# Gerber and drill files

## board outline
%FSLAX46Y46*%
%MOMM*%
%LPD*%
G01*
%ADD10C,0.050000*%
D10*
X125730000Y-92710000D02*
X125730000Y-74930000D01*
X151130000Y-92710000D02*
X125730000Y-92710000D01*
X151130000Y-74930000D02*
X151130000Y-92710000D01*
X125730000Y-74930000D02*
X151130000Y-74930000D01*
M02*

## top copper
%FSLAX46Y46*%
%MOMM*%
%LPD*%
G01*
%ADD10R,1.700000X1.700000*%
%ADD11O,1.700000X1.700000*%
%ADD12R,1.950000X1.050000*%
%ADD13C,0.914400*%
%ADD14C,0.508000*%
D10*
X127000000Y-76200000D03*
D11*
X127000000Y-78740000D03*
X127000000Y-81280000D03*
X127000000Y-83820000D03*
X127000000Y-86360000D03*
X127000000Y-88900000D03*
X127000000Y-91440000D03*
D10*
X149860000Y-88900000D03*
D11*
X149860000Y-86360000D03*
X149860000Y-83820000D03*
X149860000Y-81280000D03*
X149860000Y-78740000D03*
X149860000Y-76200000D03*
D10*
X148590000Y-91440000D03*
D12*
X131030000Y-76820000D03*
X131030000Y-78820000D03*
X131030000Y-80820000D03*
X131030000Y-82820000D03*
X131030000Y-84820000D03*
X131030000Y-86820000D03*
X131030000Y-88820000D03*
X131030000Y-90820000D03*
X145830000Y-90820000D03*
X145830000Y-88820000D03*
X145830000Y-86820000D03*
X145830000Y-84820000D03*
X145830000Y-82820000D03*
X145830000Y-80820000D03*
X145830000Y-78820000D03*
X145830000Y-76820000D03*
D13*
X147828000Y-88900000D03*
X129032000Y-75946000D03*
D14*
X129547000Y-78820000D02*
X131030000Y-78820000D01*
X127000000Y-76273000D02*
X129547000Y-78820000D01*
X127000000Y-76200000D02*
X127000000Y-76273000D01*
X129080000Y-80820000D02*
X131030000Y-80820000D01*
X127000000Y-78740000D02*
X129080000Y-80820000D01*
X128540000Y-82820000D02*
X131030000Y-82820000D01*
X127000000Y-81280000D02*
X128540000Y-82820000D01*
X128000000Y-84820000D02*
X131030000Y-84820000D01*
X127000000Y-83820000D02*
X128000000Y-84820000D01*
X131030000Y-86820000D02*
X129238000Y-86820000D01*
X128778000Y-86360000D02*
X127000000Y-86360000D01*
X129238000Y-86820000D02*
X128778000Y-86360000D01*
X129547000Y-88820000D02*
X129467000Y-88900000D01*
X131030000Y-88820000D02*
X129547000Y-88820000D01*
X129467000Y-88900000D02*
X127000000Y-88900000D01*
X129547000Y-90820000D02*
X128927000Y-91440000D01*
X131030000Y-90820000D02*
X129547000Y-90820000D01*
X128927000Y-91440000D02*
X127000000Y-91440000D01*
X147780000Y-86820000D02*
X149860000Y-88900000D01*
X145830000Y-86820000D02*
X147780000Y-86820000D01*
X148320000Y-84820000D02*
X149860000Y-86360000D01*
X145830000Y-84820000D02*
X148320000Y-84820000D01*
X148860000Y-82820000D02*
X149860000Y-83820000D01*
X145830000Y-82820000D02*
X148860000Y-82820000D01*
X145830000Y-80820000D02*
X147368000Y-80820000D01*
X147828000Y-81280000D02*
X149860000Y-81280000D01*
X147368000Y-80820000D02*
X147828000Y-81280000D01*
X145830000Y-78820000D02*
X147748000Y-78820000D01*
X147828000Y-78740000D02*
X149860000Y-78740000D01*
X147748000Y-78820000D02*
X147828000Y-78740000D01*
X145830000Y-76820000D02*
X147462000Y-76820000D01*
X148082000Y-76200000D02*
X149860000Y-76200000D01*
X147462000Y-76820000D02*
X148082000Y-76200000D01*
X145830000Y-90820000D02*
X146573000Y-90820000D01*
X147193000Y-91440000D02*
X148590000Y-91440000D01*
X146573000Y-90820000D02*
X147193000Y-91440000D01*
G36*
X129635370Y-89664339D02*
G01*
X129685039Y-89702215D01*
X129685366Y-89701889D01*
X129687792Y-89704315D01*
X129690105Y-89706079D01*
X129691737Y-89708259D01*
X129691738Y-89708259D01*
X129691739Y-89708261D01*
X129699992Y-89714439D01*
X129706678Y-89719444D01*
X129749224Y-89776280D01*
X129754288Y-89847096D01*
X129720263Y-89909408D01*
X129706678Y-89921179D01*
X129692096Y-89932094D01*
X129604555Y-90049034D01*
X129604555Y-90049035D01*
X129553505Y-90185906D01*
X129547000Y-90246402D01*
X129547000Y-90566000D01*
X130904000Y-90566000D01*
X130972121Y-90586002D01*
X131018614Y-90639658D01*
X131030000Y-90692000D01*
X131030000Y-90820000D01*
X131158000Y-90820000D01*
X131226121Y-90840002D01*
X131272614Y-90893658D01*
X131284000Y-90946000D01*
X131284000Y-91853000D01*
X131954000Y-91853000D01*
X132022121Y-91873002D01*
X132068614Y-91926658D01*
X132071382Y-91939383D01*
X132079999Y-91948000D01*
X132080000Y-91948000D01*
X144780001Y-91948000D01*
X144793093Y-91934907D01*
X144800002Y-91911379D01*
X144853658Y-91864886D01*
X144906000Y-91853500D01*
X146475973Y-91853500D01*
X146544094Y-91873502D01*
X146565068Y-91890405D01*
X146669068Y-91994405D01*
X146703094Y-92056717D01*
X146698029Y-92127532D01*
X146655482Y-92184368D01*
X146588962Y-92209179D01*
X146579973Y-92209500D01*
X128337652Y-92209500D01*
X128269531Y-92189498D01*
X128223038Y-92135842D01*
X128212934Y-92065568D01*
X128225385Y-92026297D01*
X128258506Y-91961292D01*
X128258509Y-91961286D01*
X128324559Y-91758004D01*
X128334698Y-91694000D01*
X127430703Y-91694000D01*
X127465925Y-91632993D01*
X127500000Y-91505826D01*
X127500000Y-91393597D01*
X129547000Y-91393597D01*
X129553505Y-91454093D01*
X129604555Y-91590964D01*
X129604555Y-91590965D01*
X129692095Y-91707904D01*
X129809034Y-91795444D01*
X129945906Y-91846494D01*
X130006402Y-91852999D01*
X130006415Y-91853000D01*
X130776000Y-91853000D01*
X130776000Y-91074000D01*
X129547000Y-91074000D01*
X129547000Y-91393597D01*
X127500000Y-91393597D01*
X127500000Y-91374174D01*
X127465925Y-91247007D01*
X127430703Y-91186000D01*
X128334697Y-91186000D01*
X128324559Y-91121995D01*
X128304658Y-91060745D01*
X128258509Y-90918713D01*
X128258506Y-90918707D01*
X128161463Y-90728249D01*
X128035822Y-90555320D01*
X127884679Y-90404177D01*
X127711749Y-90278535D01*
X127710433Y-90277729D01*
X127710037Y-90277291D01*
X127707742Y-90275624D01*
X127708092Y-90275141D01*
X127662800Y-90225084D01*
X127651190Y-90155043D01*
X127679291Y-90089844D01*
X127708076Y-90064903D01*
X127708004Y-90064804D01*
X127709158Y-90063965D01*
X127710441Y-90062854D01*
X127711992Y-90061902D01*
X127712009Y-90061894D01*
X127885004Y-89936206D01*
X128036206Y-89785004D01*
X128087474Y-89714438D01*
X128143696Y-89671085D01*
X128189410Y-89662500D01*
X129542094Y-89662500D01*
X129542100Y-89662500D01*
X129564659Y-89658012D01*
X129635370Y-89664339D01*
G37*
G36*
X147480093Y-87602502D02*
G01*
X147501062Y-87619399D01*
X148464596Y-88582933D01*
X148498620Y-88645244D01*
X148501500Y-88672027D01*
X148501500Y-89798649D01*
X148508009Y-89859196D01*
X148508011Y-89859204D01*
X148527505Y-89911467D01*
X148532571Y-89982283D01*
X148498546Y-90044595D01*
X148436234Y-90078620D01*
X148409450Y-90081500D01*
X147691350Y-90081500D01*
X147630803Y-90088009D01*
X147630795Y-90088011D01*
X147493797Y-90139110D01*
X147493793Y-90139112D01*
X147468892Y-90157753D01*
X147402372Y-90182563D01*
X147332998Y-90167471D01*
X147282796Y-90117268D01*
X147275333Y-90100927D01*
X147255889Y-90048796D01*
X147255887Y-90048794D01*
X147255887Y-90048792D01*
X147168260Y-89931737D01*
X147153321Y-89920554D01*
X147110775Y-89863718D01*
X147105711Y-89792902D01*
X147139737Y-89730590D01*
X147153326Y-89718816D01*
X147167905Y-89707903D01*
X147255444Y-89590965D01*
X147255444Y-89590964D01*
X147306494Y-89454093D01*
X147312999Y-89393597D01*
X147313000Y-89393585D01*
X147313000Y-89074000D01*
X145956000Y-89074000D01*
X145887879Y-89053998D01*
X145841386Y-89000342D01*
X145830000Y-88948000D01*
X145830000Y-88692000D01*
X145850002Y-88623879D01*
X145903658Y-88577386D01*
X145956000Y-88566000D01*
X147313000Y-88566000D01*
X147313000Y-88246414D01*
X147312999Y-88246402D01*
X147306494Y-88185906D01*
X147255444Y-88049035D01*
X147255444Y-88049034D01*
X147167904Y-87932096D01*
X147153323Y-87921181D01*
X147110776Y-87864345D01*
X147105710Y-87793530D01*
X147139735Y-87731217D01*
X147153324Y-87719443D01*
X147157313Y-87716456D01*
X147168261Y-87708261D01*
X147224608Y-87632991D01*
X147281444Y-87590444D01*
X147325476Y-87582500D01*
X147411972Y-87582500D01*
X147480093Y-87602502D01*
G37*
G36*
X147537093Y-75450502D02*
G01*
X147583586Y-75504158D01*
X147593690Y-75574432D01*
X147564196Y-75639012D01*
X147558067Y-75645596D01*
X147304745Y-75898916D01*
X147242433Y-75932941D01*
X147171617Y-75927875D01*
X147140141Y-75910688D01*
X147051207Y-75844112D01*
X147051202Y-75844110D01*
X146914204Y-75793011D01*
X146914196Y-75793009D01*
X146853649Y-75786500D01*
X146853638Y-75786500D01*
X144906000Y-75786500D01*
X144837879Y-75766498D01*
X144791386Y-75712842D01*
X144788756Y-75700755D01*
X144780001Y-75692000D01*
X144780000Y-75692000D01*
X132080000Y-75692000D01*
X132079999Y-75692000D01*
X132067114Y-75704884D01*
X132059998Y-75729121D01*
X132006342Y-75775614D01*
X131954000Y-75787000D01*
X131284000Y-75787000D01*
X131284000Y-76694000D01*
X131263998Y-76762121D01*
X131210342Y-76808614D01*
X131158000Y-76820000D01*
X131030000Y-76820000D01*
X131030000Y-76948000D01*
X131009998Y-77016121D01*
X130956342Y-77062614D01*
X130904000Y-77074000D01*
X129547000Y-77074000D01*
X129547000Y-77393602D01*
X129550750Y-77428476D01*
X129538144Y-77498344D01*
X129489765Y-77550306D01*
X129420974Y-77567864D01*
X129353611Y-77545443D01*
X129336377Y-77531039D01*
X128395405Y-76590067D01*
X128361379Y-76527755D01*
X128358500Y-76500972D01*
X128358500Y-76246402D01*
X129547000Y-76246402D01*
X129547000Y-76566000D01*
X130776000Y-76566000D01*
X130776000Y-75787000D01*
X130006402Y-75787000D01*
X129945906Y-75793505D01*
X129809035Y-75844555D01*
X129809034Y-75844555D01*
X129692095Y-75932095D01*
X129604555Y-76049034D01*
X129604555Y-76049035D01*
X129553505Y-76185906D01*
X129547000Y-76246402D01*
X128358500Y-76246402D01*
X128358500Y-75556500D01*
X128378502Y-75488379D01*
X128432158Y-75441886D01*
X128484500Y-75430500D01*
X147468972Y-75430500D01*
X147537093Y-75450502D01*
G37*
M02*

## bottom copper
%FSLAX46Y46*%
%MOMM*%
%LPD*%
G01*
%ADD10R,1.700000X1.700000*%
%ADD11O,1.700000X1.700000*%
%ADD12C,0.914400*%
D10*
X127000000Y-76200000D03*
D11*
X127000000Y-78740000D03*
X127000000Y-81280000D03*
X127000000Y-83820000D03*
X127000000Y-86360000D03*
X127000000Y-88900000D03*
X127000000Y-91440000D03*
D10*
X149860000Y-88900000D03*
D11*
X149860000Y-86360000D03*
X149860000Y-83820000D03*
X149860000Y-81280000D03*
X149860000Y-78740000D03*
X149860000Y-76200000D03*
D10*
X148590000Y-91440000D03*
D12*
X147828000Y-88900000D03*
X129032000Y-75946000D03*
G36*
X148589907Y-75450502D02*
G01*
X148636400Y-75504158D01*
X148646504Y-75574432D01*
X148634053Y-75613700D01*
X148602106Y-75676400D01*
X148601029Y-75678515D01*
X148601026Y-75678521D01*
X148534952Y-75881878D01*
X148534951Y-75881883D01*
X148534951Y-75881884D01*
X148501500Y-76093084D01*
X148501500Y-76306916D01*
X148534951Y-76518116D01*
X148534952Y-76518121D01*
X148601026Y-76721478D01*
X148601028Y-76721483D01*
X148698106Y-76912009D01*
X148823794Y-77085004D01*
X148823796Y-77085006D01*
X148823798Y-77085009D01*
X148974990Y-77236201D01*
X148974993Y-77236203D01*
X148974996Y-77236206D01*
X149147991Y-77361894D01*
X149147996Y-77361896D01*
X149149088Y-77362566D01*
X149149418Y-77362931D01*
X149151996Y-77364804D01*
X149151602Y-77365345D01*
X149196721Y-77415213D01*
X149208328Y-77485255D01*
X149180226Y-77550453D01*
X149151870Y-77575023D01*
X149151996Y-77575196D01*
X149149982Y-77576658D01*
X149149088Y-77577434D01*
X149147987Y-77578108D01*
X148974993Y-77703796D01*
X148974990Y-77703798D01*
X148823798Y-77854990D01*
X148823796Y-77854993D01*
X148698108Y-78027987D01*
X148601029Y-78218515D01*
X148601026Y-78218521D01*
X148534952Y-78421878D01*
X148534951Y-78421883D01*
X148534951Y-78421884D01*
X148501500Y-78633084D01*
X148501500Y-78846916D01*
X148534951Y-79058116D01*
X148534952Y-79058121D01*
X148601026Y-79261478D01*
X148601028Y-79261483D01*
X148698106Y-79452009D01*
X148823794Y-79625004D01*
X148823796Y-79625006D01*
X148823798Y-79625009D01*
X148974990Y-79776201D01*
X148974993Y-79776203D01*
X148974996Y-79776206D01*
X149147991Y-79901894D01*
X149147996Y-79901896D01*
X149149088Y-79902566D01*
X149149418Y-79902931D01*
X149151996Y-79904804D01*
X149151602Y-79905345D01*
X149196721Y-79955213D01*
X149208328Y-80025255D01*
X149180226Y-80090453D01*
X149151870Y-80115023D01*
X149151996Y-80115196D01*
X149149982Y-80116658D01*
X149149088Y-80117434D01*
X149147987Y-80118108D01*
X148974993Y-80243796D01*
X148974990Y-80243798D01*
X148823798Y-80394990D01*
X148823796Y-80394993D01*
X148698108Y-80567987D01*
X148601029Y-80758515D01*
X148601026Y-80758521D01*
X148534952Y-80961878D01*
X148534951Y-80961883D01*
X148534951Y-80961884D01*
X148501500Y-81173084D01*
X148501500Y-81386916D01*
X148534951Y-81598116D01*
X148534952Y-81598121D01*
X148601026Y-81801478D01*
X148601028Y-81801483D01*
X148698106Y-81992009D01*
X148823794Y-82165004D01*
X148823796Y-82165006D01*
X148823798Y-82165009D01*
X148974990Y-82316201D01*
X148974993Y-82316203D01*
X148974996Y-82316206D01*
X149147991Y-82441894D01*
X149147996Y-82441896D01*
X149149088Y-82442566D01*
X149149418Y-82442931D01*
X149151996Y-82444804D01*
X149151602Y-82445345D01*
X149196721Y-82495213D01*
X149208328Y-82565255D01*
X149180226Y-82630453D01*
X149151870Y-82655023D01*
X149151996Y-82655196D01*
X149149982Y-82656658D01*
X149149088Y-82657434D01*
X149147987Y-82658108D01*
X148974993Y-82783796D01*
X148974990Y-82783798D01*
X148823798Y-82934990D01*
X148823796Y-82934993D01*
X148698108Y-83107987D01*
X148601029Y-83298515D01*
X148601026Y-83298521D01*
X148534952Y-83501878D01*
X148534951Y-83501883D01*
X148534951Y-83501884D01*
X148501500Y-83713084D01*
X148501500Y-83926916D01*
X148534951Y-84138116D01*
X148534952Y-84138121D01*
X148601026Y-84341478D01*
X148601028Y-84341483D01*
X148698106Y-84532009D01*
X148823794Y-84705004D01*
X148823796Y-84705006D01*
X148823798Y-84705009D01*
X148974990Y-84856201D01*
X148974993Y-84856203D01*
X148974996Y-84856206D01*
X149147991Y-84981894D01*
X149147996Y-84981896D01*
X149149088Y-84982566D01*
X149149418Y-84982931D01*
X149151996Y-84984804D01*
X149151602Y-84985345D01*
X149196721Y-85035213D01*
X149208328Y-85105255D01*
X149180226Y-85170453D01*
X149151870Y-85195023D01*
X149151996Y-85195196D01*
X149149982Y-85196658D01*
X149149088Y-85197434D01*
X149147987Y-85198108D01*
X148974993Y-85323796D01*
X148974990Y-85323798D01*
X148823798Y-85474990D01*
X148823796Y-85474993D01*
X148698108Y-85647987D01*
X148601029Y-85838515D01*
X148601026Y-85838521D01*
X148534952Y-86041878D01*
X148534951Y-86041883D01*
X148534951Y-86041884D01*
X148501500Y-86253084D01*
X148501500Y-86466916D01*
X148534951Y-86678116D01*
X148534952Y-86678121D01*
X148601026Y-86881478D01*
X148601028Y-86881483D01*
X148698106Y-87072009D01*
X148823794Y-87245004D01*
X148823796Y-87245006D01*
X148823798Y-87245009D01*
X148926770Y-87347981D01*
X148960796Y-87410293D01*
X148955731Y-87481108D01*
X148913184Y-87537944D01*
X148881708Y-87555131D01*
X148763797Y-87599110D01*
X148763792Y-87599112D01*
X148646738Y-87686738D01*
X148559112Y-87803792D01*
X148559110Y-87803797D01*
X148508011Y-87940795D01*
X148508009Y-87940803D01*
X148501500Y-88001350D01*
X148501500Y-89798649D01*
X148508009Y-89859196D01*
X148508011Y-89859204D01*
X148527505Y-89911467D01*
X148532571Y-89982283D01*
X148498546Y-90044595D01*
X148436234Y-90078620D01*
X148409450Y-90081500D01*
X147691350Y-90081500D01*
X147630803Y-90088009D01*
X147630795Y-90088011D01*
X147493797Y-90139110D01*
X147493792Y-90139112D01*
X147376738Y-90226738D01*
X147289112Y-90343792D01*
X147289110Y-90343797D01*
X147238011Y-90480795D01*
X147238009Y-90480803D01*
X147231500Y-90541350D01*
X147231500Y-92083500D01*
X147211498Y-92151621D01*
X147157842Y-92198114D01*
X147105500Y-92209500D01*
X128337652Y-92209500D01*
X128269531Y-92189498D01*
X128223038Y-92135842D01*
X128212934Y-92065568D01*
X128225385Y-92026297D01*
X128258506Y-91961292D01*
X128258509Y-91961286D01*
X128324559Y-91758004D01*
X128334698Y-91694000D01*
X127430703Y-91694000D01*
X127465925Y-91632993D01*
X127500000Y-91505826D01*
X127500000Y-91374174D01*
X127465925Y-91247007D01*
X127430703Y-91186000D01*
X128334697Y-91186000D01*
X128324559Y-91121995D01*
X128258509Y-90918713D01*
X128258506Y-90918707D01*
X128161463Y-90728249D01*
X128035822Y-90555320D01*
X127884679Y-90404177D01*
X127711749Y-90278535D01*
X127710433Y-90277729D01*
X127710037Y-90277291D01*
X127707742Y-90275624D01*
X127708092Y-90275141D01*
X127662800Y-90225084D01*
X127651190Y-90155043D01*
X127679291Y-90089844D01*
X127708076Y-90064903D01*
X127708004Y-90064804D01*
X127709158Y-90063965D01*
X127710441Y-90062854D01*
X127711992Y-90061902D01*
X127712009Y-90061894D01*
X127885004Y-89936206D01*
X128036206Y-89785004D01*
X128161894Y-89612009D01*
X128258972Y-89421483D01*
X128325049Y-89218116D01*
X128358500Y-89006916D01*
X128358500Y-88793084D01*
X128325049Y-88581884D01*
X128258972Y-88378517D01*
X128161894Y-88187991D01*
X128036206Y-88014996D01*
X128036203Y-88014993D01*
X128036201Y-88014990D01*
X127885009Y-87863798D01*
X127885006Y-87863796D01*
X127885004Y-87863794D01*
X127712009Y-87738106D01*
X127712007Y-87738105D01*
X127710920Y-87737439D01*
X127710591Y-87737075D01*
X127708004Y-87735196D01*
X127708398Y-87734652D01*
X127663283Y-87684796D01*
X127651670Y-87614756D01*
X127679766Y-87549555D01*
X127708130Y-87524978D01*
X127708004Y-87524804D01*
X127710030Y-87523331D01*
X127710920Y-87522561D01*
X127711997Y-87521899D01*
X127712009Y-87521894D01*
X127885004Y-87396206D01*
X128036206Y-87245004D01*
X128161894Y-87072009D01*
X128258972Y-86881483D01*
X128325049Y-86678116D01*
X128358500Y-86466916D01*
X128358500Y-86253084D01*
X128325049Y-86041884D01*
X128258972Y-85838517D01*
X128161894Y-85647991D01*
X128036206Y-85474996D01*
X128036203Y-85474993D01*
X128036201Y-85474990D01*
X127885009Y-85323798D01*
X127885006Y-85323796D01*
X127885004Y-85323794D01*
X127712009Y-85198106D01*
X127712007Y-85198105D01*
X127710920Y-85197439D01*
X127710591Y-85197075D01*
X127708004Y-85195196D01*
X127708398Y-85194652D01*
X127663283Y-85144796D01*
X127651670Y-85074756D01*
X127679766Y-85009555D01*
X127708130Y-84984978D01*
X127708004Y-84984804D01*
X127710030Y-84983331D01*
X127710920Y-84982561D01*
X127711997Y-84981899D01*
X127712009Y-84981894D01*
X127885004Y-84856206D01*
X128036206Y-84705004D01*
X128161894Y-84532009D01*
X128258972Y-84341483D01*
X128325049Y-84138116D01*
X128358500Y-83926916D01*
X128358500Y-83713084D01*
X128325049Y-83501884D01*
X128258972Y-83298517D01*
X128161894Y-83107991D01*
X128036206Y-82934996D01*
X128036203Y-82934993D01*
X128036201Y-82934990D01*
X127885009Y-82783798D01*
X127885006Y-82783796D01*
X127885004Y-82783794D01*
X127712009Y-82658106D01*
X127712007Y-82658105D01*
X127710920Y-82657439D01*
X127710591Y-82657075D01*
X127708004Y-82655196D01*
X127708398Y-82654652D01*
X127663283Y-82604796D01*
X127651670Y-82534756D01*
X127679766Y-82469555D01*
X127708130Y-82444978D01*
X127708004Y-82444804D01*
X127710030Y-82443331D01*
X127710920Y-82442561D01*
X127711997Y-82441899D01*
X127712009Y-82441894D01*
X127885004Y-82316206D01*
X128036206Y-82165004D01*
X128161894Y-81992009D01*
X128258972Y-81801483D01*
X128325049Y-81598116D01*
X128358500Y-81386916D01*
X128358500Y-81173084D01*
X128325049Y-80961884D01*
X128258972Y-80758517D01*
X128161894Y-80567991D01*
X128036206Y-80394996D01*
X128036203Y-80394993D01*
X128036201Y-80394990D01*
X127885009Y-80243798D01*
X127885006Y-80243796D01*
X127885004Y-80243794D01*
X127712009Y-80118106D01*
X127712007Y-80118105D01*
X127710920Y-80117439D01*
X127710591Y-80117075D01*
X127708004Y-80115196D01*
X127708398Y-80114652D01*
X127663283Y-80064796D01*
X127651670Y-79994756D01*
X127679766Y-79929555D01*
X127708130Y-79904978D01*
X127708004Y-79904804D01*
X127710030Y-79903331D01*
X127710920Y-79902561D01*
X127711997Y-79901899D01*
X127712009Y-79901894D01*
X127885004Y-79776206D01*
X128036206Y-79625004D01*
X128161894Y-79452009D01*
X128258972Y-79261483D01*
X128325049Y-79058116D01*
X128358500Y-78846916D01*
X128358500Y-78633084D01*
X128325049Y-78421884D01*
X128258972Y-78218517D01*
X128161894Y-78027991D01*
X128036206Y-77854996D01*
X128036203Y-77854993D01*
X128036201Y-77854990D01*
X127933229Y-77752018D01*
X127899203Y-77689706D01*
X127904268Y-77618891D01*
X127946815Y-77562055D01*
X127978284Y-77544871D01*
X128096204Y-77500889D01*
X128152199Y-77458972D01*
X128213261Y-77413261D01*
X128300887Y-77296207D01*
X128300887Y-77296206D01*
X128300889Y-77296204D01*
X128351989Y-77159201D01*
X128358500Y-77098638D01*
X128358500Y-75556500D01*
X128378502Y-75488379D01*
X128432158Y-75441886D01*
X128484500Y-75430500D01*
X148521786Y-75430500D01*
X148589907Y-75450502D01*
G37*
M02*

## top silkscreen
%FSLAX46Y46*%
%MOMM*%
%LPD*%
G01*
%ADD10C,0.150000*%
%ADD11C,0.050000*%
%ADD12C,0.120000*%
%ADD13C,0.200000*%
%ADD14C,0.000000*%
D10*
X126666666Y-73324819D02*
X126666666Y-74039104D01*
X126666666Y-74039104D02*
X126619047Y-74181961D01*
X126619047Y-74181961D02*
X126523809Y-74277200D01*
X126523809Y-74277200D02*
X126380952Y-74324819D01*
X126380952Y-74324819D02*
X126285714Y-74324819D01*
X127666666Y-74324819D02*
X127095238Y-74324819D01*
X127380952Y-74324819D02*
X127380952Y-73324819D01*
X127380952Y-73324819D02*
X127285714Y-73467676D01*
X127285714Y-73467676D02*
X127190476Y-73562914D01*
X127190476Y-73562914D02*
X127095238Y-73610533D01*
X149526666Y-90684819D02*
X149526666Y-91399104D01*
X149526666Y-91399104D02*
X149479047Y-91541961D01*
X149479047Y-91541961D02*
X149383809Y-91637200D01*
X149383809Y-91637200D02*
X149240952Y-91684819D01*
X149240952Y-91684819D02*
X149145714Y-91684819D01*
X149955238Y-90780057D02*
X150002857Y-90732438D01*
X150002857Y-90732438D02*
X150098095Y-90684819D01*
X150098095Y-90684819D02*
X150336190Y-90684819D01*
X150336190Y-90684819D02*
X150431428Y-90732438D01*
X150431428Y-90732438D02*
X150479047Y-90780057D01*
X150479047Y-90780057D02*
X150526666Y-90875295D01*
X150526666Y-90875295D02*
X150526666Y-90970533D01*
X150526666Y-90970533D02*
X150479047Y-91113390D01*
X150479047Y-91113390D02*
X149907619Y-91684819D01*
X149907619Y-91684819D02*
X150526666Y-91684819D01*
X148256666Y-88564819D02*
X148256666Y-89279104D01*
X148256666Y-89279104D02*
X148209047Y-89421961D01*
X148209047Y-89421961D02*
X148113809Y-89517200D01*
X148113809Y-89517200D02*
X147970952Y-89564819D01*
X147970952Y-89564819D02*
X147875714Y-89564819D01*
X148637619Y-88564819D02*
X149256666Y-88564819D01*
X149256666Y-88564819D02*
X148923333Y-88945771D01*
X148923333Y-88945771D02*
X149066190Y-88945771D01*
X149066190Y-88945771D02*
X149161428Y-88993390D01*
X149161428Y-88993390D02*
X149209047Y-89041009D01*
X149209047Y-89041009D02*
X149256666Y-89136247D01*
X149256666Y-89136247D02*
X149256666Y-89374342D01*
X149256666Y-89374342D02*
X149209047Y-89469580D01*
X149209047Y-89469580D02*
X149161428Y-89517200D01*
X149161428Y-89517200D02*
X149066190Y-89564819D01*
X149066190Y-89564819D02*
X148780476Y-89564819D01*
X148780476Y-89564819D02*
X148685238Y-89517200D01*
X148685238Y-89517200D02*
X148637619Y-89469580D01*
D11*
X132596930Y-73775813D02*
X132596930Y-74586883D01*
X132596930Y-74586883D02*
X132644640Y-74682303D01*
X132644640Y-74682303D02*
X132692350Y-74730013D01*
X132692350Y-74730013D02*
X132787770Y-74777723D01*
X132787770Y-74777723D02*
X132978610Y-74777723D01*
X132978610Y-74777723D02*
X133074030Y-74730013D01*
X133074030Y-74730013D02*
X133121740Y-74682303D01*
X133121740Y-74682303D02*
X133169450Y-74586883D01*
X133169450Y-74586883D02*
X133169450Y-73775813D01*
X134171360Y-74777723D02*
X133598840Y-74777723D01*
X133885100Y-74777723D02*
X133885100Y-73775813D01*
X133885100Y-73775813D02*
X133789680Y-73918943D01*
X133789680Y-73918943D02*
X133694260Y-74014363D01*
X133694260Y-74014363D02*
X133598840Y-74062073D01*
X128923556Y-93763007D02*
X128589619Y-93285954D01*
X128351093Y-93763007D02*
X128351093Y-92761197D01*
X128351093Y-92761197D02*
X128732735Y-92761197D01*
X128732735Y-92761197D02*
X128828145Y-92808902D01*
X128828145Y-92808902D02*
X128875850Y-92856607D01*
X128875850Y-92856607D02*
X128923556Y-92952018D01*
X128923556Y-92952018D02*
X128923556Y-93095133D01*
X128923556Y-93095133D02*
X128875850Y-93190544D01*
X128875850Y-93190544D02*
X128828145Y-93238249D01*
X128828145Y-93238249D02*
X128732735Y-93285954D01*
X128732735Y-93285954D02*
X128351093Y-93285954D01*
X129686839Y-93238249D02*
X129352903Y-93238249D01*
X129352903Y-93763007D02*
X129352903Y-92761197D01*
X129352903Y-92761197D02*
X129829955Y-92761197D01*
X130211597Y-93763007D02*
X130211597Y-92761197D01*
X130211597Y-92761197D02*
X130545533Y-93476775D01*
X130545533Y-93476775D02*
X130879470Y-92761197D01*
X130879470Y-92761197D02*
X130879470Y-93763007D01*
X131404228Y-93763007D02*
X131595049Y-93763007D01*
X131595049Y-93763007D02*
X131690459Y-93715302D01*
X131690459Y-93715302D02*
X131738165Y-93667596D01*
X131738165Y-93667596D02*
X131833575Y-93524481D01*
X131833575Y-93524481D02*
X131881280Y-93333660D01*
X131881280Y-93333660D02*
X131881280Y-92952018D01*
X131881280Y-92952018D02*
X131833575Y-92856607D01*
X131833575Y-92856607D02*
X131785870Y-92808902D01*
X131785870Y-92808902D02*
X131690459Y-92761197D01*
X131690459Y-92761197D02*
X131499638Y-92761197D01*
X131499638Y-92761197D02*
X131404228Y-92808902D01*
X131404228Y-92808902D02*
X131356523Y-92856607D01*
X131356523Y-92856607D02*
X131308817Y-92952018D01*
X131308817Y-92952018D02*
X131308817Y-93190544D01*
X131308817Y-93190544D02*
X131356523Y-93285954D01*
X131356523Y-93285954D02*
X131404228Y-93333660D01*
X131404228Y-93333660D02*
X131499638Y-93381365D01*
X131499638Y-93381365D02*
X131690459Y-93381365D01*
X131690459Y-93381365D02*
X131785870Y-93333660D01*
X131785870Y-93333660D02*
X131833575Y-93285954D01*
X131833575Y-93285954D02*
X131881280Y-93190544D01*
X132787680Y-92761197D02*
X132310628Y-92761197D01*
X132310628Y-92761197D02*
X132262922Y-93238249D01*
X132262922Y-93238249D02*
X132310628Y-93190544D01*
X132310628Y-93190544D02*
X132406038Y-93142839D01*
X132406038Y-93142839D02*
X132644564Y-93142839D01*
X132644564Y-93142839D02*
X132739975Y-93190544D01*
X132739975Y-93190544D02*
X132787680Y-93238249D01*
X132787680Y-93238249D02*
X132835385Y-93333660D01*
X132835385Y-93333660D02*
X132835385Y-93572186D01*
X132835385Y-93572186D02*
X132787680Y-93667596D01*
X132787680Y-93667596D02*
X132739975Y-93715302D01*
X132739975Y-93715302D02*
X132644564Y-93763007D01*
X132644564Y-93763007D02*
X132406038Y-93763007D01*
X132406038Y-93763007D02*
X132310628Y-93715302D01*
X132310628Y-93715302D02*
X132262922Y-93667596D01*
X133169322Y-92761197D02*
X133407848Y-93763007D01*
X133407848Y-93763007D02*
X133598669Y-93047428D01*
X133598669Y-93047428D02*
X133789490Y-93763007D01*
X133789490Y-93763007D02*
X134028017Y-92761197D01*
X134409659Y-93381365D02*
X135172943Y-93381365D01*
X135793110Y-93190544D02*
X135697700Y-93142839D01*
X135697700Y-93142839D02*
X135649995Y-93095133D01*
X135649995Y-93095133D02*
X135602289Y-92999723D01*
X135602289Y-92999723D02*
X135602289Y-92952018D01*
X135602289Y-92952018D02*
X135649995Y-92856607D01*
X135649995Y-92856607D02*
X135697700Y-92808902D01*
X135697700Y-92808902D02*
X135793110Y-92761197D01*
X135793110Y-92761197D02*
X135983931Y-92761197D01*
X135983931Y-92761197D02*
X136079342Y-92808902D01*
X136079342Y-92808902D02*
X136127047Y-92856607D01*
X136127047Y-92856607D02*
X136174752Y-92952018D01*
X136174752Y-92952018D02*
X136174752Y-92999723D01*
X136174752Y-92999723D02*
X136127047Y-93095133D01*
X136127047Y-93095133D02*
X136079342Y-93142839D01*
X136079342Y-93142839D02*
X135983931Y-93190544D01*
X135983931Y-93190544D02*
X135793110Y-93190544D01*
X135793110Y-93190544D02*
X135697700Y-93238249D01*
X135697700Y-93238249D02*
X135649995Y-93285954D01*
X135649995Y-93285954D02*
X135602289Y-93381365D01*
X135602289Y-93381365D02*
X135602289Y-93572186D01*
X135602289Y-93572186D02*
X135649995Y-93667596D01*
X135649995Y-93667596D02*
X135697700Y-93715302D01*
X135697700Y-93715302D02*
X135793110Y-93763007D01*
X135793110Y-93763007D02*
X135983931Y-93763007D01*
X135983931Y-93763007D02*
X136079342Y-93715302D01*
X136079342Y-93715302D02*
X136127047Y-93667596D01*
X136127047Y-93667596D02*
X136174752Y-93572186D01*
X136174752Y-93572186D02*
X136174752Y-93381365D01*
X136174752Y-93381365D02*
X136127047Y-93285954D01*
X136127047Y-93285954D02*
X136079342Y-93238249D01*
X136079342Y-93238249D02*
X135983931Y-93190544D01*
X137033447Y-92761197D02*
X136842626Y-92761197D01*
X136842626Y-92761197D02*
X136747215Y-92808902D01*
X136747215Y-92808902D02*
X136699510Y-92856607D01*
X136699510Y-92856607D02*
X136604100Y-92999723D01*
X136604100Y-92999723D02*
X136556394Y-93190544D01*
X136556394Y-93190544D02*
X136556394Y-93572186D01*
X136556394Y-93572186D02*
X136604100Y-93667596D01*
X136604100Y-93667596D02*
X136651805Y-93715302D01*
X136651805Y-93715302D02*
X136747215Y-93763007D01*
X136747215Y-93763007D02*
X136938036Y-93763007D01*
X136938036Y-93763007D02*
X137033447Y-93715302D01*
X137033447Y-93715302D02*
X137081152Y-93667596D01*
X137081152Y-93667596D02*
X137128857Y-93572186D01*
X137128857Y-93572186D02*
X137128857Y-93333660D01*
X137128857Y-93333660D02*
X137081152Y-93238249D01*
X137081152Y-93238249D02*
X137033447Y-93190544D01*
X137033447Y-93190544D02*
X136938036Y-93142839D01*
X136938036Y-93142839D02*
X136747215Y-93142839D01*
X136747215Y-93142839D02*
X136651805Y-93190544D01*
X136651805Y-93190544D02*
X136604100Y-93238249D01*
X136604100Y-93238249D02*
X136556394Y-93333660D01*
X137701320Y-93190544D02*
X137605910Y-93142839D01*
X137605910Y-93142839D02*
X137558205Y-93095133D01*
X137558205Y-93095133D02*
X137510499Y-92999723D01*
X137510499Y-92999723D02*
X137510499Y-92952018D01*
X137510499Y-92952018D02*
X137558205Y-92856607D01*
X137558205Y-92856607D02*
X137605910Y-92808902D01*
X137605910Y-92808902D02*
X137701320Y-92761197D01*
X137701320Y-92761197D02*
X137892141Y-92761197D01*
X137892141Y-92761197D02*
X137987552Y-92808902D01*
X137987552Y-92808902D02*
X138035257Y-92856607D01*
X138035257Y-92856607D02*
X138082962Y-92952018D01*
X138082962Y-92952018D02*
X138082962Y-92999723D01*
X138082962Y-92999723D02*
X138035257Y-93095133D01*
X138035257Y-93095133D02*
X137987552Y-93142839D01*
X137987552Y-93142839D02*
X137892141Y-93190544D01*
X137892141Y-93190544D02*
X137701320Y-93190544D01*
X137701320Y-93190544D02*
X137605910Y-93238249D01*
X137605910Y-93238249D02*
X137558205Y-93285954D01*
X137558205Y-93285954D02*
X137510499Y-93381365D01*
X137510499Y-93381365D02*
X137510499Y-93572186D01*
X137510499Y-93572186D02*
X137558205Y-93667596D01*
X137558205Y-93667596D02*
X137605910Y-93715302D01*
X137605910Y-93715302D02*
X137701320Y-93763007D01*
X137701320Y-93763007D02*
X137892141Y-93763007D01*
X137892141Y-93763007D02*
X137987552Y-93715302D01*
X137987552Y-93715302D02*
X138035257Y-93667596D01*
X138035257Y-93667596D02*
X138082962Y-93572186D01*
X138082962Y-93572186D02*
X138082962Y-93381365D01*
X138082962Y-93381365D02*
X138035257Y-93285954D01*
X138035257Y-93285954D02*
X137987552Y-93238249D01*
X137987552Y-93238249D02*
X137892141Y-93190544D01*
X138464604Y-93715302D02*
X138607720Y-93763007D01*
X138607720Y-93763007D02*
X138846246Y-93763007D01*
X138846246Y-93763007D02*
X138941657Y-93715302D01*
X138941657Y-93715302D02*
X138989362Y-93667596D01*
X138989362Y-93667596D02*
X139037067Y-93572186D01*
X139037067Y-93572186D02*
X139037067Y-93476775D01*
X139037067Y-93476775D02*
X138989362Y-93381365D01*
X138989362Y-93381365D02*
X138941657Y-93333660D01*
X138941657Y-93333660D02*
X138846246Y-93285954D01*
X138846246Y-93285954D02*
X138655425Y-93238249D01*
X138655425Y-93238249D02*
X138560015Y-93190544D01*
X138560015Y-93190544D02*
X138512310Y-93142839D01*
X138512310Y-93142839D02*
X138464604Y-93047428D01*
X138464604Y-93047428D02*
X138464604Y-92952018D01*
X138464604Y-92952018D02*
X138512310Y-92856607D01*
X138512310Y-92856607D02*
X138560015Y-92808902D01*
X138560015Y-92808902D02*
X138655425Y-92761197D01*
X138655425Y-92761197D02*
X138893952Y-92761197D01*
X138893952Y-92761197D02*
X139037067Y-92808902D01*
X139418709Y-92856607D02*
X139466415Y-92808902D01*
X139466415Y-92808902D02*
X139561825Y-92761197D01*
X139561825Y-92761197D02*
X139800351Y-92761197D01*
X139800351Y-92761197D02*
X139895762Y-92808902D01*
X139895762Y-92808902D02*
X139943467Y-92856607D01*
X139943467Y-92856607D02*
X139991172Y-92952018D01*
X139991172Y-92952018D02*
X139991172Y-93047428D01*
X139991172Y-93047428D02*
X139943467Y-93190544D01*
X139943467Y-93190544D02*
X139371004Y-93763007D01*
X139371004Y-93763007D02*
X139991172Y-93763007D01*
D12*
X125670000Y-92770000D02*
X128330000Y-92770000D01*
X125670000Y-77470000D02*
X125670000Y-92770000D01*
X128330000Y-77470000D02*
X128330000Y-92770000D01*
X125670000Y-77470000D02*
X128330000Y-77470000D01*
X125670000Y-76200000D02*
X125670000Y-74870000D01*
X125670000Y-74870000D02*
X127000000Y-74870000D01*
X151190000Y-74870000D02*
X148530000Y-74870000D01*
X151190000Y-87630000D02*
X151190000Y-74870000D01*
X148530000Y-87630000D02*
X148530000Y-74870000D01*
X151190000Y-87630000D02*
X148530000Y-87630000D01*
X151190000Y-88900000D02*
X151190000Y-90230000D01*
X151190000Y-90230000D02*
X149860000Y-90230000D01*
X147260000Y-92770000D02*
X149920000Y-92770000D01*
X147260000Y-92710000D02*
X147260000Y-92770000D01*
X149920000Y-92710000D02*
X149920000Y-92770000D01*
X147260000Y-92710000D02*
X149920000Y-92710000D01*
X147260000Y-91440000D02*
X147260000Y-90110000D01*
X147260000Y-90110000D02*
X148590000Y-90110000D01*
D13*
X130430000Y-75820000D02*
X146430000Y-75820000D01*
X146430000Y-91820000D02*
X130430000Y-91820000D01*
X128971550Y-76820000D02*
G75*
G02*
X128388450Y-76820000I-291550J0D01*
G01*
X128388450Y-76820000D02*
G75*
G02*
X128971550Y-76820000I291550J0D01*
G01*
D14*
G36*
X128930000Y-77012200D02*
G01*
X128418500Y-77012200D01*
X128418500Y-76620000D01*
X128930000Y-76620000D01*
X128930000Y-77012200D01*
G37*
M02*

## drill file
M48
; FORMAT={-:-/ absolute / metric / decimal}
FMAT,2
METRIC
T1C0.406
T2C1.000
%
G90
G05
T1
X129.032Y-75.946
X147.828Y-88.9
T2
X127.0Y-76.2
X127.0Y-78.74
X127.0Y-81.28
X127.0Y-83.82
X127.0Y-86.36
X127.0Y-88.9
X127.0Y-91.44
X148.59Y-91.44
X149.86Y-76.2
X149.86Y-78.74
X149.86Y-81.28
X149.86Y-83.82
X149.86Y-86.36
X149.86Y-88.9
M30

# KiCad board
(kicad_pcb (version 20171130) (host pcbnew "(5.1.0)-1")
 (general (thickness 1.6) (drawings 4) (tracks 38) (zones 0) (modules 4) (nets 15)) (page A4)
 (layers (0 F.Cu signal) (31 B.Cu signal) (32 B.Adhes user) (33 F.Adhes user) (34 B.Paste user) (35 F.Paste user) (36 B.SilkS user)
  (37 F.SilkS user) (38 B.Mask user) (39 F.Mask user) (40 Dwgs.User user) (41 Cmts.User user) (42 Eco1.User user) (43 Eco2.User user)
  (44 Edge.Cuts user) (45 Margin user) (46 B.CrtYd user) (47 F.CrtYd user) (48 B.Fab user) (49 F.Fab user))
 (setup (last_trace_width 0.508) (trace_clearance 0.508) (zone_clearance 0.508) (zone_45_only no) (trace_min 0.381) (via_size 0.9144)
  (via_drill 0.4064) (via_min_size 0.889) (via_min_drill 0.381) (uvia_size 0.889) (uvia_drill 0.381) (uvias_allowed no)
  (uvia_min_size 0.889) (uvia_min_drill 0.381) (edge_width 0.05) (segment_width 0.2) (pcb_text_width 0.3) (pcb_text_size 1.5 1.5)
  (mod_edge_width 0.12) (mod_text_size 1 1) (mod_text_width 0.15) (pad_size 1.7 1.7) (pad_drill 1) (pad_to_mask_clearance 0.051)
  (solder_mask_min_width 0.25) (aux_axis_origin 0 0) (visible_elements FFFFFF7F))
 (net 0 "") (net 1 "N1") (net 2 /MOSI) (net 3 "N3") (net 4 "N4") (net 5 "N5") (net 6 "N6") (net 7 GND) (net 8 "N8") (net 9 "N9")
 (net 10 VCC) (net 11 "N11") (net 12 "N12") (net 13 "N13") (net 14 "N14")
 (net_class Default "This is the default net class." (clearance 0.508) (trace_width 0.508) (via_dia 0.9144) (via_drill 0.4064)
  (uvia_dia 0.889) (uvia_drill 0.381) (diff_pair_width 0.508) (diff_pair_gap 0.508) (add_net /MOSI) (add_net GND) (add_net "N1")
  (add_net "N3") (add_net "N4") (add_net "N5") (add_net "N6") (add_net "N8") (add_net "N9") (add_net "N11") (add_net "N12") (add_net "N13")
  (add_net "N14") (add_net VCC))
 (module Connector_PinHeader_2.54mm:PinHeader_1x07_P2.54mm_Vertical (layer F.Cu) (at 127 76.2)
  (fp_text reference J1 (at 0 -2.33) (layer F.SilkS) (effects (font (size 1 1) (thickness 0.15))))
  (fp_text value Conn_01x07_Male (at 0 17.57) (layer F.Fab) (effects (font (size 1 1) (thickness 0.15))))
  (fp_line (start -1.33 16.57) (end 1.33 16.57) (layer F.SilkS) (width 0.12))
  (fp_line (start -1.33 1.27) (end -1.33 16.57) (layer F.SilkS) (width 0.12))
  (fp_line (start 1.33 1.27) (end 1.33 16.57) (layer F.SilkS) (width 0.12))
  (fp_line (start -1.33 1.27) (end 1.33 1.27) (layer F.SilkS) (width 0.12))
  (fp_line (start -1.33 0) (end -1.33 -1.33) (layer F.SilkS) (width 0.12))
  (fp_line (start -1.33 -1.33) (end 0 -1.33) (layer F.SilkS) (width 0.12))
  (pad 1 thru_hole rect (at 0 0) (size 1.7 1.7) (drill 1) (layers *.Cu *.Mask) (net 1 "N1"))
  (pad 2 thru_hole oval (at 0 2.54) (size 1.7 1.7) (drill 1) (layers *.Cu *.Mask) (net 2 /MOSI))
  (pad 3 thru_hole oval (at 0 5.08) (size 1.7 1.7) (drill 1) (layers *.Cu *.Mask) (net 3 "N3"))
  (pad 4 thru_hole oval (at 0 7.62) (size 1.7 1.7) (drill 1) (layers *.Cu *.Mask) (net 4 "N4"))
  (pad 5 thru_hole oval (at 0 10.16) (size 1.7 1.7) (drill 1) (layers *.Cu *.Mask) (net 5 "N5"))
  (pad 6 thru_hole oval (at 0 12.7) (size 1.7 1.7) (drill 1) (layers *.Cu *.Mask) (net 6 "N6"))
  (pad 7 thru_hole oval (at 0 15.24) (size 1.7 1.7) (drill 1) (layers *.Cu *.Mask) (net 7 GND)))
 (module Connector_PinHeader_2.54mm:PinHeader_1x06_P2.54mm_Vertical (layer F.Cu) (at 149.86 88.9 180)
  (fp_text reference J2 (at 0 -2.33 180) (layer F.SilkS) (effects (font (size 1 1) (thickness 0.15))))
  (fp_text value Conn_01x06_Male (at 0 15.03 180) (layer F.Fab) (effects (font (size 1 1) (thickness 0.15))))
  (fp_line (start -1.33 14.03) (end 1.33 14.03) (layer F.SilkS) (width 0.12))
  (fp_line (start -1.33 1.27) (end -1.33 14.03) (layer F.SilkS) (width 0.12))
  (fp_line (start 1.33 1.27) (end 1.33 14.03) (layer F.SilkS) (width 0.12))
  (fp_line (start -1.33 1.27) (end 1.33 1.27) (layer F.SilkS) (width 0.12))
  (fp_line (start -1.33 0) (end -1.33 -1.33) (layer F.SilkS) (width 0.12))
  (fp_line (start -1.33 -1.33) (end 0 -1.33) (layer F.SilkS) (width 0.12))
  (pad 1 thru_hole rect (at 0 0 180) (size 1.7 1.7) (drill 1) (layers *.Cu *.Mask) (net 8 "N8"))
  (pad 2 thru_hole oval (at 0 2.54 180) (size 1.7 1.7) (drill 1) (layers *.Cu *.Mask) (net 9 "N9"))
  (pad 3 thru_hole oval (at 0 5.08 180) (size 1.7 1.7) (drill 1) (layers *.Cu *.Mask) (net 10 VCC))
  (pad 4 thru_hole oval (at 0 7.62 180) (size 1.7 1.7) (drill 1) (layers *.Cu *.Mask) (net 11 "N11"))
  (pad 5 thru_hole oval (at 0 10.16 180) (size 1.7 1.7) (drill 1) (layers *.Cu *.Mask) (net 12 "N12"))
  (pad 6 thru_hole oval (at 0 12.7 180) (size 1.7 1.7) (drill 1) (layers *.Cu *.Mask) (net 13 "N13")))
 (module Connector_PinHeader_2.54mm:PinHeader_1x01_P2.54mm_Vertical (layer F.Cu) (at 148.59 91.44)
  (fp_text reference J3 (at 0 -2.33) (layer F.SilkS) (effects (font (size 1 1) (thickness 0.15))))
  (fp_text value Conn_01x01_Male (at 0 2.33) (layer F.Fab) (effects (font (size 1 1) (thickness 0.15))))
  (fp_line (start -1.33 1.33) (end 1.33 1.33) (layer F.SilkS) (width 0.12))
  (fp_line (start -1.33 1.27) (end -1.33 1.33) (layer F.SilkS) (width 0.12))
  (fp_line (start 1.33 1.27) (end 1.33 1.33) (layer F.SilkS) (width 0.12))
  (fp_line (start -1.33 1.27) (end 1.33 1.27) (layer F.SilkS) (width 0.12))
  (fp_line (start -1.33 0) (end -1.33 -1.33) (layer F.SilkS) (width 0.12))
  (fp_line (start -1.33 -1.33) (end 0 -1.33) (layer F.SilkS) (width 0.12))
  (pad 1 thru_hole rect (at 0 0) (size 1.7 1.7) (drill 1) (layers *.Cu *.Mask) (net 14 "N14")))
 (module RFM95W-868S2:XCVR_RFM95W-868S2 (layer F.Cu) (at 138.43 83.82)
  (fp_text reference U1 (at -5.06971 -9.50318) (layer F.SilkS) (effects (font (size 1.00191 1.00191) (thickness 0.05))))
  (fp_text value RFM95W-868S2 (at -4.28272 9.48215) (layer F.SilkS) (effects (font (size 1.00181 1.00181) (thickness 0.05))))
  (fp_line (start -8 -8) (end 8 -8) (layer F.SilkS) (width 0.2)) (fp_line (start 8 8) (end -8 8) (layer F.SilkS) (width 0.2))
  (fp_circle (center -9.75 -7) (end -9.45845 -7) (layer F.SilkS) (width 0.2))
  (fp_poly (pts (xy -10.0115 -7.2) (xy -9.5 -7.2) (xy -9.5 -6.8078) (xy -10.0115 -6.8078)) (layer F.SilkS) (width 0))
  (pad 1 smd rect (at -7.4 -7) (size 1.95 1.05) (layers F.Cu F.Paste F.Mask) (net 7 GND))
  (pad 2 smd rect (at -7.4 -5) (size 1.95 1.05) (layers F.Cu F.Paste F.Mask) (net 1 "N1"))
  (pad 3 smd rect (at -7.4 -3) (size 1.95 1.05) (layers F.Cu F.Paste F.Mask) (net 2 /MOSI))
  (pad 4 smd rect (at -7.4 -1) (size 1.95 1.05) (layers F.Cu F.Paste F.Mask) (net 3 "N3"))
  (pad 5 smd rect (at -7.4 1) (size 1.95 1.05) (layers F.Cu F.Paste F.Mask) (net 4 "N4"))
  (pad 6 smd rect (at -7.4 3) (size 1.95 1.05) (layers F.Cu F.Paste F.Mask) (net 5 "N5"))
  (pad 7 smd rect (at -7.4 5) (size 1.95 1.05) (layers F.Cu F.Paste F.Mask) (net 6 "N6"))
  (pad 8 smd rect (at -7.4 7) (size 1.95 1.05) (layers F.Cu F.Paste F.Mask) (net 7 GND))
  (pad 9 smd rect (at 7.4 7 180) (size 1.95 1.05) (layers F.Cu F.Paste F.Mask) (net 14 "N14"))
  (pad 10 smd rect (at 7.4 5 180) (size 1.95 1.05) (layers F.Cu F.Paste F.Mask) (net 7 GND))
  (pad 11 smd rect (at 7.4 3 180) (size 1.95 1.05) (layers F.Cu F.Paste F.Mask) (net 8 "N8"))
  (pad 12 smd rect (at 7.4 1 180) (size 1.95 1.05) (layers F.Cu F.Paste F.Mask) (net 9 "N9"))
  (pad 13 smd rect (at 7.4 -1 180) (size 1.95 1.05) (layers F.Cu F.Paste F.Mask) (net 10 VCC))
  (pad 14 smd rect (at 7.4 -3 180) (size 1.95 1.05) (layers F.Cu F.Paste F.Mask) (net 11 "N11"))
  (pad 15 smd rect (at 7.4 -5 180) (size 1.95 1.05) (layers F.Cu F.Paste F.Mask) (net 12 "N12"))
  (pad 16 smd rect (at 7.4 -7 180) (size 1.95 1.05) (layers F.Cu F.Paste F.Mask) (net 13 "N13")))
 (gr_line (start 125.73 92.71) (end 125.73 74.93) (layer Edge.Cuts) (width 0.05))
 (gr_line (start 151.13 92.71) (end 125.73 92.71) (layer Edge.Cuts) (width 0.05))
 (gr_line (start 151.13 74.93) (end 151.13 92.71) (layer Edge.Cuts) (width 0.05))
 (gr_line (start 125.73 74.93) (end 151.13 74.93) (layer Edge.Cuts) (width 0.05))
 (via (at 147.828 88.9) (size 0.9144) (drill 0.4064) (layers F.Cu B.Cu) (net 7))
 (segment (start 129.547 78.82) (end 131.03 78.82) (width 0.508) (layer F.Cu) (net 1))
 (segment (start 127 76.273) (end 129.547 78.82) (width 0.508) (layer F.Cu) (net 1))
 (segment (start 127 76.2) (end 127 76.273) (width 0.508) (layer F.Cu) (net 1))
 (segment (start 129.08 80.82) (end 131.03 80.82) (width 0.508) (layer F.Cu) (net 2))
 (segment (start 127 78.74) (end 129.08 80.82) (width 0.508) (layer F.Cu) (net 2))
 (segment (start 128.54 82.82) (end 131.03 82.82) (width 0.508) (layer F.Cu) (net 3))
 (segment (start 127 81.28) (end 128.54 82.82) (width 0.508) (layer F.Cu) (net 3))
 (segment (start 128 84.82) (end 131.03 84.82) (width 0.508) (layer F.Cu) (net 4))
 (segment (start 127 83.82) (end 128 84.82) (width 0.508) (layer F.Cu) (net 4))
 (segment (start 131.03 86.82) (end 129.238 86.82) (width 0.508) (layer F.Cu) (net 5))
 (segment (start 128.778 86.36) (end 127 86.36) (width 0.508) (layer F.Cu) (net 5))
 (segment (start 129.238 86.82) (end 128.778 86.36) (width 0.508) (layer F.Cu) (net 5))
 (segment (start 129.547 88.82) (end 129.467 88.9) (width 0.508) (layer F.Cu) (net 6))
 (segment (start 131.03 88.82) (end 129.547 88.82) (width 0.508) (layer F.Cu) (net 6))
 (segment (start 129.467 88.9) (end 127 88.9) (width 0.508) (layer F.Cu) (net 6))
 (segment (start 129.547 90.82) (end 128.927 91.44) (width 0.508) (layer F.Cu) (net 7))
 (segment (start 131.03 90.82) (end 129.547 90.82) (width 0.508) (layer F.Cu) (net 7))
 (segment (start 128.927 91.44) (end 127 91.44) (width 0.508) (layer F.Cu) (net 7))
 (via (at 129.032 75.946) (size 0.9144) (drill 0.4064) (layers F.Cu B.Cu) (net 7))
 (segment (start 147.78 86.82) (end 149.86 88.9) (width 0.508) (layer F.Cu) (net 8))
 (segment (start 145.83 86.82) (end 147.78 86.82) (width 0.508) (layer F.Cu) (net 8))
 (segment (start 148.32 84.82) (end 149.86 86.36) (width 0.508) (layer F.Cu) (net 9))
 (segment (start 145.83 84.82) (end 148.32 84.82) (width 0.508) (layer F.Cu) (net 9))
 (segment (start 148.86 82.82) (end 149.86 83.82) (width 0.508) (layer F.Cu) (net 10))
 (segment (start 145.83 82.82) (end 148.86 82.82) (width 0.508) (layer F.Cu) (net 10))
 (segment (start 145.83 80.82) (end 147.368 80.82) (width 0.508) (layer F.Cu) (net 11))
 (segment (start 147.828 81.28) (end 149.86 81.28) (width 0.508) (layer F.Cu) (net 11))
 (segment (start 147.368 80.82) (end 147.828 81.28) (width 0.508) (layer F.Cu) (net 11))
 (segment (start 145.83 78.82) (end 147.748 78.82) (width 0.508) (layer F.Cu) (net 12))
 (segment (start 147.828 78.74) (end 149.86 78.74) (width 0.508) (layer F.Cu) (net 12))
 (segment (start 147.748 78.82) (end 147.828 78.74) (width 0.508) (layer F.Cu) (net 12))
 (segment (start 145.83 76.82) (end 147.462 76.82) (width 0.508) (layer F.Cu) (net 13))
 (segment (start 148.082 76.2) (end 149.86 76.2) (width 0.508) (layer F.Cu) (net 13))
 (segment (start 147.462 76.82) (end 148.082 76.2) (width 0.508) (layer F.Cu) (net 13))
 (segment (start 145.83 90.82) (end 146.573 90.82) (width 0.508) (layer F.Cu) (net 14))
 (segment (start 147.193 91.44) (end 148.59 91.44) (width 0.508) (layer F.Cu) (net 14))
 (segment (start 146.573 90.82) (end 147.193 91.44) (width 0.508) (layer F.Cu) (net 14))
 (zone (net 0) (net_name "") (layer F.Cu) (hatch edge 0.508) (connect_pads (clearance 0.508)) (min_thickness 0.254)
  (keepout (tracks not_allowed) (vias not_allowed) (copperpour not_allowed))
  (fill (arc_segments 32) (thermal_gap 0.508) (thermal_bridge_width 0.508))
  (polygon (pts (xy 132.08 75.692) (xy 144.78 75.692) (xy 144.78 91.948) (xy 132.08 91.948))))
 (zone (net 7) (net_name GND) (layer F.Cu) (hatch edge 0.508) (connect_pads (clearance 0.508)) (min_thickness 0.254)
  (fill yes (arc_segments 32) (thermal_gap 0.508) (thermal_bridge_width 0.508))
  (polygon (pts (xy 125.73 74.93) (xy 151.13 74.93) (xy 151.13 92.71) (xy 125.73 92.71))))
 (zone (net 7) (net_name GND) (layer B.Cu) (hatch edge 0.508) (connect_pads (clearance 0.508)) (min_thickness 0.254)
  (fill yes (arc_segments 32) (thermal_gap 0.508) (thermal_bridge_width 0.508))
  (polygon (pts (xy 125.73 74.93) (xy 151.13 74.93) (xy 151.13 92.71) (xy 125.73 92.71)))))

